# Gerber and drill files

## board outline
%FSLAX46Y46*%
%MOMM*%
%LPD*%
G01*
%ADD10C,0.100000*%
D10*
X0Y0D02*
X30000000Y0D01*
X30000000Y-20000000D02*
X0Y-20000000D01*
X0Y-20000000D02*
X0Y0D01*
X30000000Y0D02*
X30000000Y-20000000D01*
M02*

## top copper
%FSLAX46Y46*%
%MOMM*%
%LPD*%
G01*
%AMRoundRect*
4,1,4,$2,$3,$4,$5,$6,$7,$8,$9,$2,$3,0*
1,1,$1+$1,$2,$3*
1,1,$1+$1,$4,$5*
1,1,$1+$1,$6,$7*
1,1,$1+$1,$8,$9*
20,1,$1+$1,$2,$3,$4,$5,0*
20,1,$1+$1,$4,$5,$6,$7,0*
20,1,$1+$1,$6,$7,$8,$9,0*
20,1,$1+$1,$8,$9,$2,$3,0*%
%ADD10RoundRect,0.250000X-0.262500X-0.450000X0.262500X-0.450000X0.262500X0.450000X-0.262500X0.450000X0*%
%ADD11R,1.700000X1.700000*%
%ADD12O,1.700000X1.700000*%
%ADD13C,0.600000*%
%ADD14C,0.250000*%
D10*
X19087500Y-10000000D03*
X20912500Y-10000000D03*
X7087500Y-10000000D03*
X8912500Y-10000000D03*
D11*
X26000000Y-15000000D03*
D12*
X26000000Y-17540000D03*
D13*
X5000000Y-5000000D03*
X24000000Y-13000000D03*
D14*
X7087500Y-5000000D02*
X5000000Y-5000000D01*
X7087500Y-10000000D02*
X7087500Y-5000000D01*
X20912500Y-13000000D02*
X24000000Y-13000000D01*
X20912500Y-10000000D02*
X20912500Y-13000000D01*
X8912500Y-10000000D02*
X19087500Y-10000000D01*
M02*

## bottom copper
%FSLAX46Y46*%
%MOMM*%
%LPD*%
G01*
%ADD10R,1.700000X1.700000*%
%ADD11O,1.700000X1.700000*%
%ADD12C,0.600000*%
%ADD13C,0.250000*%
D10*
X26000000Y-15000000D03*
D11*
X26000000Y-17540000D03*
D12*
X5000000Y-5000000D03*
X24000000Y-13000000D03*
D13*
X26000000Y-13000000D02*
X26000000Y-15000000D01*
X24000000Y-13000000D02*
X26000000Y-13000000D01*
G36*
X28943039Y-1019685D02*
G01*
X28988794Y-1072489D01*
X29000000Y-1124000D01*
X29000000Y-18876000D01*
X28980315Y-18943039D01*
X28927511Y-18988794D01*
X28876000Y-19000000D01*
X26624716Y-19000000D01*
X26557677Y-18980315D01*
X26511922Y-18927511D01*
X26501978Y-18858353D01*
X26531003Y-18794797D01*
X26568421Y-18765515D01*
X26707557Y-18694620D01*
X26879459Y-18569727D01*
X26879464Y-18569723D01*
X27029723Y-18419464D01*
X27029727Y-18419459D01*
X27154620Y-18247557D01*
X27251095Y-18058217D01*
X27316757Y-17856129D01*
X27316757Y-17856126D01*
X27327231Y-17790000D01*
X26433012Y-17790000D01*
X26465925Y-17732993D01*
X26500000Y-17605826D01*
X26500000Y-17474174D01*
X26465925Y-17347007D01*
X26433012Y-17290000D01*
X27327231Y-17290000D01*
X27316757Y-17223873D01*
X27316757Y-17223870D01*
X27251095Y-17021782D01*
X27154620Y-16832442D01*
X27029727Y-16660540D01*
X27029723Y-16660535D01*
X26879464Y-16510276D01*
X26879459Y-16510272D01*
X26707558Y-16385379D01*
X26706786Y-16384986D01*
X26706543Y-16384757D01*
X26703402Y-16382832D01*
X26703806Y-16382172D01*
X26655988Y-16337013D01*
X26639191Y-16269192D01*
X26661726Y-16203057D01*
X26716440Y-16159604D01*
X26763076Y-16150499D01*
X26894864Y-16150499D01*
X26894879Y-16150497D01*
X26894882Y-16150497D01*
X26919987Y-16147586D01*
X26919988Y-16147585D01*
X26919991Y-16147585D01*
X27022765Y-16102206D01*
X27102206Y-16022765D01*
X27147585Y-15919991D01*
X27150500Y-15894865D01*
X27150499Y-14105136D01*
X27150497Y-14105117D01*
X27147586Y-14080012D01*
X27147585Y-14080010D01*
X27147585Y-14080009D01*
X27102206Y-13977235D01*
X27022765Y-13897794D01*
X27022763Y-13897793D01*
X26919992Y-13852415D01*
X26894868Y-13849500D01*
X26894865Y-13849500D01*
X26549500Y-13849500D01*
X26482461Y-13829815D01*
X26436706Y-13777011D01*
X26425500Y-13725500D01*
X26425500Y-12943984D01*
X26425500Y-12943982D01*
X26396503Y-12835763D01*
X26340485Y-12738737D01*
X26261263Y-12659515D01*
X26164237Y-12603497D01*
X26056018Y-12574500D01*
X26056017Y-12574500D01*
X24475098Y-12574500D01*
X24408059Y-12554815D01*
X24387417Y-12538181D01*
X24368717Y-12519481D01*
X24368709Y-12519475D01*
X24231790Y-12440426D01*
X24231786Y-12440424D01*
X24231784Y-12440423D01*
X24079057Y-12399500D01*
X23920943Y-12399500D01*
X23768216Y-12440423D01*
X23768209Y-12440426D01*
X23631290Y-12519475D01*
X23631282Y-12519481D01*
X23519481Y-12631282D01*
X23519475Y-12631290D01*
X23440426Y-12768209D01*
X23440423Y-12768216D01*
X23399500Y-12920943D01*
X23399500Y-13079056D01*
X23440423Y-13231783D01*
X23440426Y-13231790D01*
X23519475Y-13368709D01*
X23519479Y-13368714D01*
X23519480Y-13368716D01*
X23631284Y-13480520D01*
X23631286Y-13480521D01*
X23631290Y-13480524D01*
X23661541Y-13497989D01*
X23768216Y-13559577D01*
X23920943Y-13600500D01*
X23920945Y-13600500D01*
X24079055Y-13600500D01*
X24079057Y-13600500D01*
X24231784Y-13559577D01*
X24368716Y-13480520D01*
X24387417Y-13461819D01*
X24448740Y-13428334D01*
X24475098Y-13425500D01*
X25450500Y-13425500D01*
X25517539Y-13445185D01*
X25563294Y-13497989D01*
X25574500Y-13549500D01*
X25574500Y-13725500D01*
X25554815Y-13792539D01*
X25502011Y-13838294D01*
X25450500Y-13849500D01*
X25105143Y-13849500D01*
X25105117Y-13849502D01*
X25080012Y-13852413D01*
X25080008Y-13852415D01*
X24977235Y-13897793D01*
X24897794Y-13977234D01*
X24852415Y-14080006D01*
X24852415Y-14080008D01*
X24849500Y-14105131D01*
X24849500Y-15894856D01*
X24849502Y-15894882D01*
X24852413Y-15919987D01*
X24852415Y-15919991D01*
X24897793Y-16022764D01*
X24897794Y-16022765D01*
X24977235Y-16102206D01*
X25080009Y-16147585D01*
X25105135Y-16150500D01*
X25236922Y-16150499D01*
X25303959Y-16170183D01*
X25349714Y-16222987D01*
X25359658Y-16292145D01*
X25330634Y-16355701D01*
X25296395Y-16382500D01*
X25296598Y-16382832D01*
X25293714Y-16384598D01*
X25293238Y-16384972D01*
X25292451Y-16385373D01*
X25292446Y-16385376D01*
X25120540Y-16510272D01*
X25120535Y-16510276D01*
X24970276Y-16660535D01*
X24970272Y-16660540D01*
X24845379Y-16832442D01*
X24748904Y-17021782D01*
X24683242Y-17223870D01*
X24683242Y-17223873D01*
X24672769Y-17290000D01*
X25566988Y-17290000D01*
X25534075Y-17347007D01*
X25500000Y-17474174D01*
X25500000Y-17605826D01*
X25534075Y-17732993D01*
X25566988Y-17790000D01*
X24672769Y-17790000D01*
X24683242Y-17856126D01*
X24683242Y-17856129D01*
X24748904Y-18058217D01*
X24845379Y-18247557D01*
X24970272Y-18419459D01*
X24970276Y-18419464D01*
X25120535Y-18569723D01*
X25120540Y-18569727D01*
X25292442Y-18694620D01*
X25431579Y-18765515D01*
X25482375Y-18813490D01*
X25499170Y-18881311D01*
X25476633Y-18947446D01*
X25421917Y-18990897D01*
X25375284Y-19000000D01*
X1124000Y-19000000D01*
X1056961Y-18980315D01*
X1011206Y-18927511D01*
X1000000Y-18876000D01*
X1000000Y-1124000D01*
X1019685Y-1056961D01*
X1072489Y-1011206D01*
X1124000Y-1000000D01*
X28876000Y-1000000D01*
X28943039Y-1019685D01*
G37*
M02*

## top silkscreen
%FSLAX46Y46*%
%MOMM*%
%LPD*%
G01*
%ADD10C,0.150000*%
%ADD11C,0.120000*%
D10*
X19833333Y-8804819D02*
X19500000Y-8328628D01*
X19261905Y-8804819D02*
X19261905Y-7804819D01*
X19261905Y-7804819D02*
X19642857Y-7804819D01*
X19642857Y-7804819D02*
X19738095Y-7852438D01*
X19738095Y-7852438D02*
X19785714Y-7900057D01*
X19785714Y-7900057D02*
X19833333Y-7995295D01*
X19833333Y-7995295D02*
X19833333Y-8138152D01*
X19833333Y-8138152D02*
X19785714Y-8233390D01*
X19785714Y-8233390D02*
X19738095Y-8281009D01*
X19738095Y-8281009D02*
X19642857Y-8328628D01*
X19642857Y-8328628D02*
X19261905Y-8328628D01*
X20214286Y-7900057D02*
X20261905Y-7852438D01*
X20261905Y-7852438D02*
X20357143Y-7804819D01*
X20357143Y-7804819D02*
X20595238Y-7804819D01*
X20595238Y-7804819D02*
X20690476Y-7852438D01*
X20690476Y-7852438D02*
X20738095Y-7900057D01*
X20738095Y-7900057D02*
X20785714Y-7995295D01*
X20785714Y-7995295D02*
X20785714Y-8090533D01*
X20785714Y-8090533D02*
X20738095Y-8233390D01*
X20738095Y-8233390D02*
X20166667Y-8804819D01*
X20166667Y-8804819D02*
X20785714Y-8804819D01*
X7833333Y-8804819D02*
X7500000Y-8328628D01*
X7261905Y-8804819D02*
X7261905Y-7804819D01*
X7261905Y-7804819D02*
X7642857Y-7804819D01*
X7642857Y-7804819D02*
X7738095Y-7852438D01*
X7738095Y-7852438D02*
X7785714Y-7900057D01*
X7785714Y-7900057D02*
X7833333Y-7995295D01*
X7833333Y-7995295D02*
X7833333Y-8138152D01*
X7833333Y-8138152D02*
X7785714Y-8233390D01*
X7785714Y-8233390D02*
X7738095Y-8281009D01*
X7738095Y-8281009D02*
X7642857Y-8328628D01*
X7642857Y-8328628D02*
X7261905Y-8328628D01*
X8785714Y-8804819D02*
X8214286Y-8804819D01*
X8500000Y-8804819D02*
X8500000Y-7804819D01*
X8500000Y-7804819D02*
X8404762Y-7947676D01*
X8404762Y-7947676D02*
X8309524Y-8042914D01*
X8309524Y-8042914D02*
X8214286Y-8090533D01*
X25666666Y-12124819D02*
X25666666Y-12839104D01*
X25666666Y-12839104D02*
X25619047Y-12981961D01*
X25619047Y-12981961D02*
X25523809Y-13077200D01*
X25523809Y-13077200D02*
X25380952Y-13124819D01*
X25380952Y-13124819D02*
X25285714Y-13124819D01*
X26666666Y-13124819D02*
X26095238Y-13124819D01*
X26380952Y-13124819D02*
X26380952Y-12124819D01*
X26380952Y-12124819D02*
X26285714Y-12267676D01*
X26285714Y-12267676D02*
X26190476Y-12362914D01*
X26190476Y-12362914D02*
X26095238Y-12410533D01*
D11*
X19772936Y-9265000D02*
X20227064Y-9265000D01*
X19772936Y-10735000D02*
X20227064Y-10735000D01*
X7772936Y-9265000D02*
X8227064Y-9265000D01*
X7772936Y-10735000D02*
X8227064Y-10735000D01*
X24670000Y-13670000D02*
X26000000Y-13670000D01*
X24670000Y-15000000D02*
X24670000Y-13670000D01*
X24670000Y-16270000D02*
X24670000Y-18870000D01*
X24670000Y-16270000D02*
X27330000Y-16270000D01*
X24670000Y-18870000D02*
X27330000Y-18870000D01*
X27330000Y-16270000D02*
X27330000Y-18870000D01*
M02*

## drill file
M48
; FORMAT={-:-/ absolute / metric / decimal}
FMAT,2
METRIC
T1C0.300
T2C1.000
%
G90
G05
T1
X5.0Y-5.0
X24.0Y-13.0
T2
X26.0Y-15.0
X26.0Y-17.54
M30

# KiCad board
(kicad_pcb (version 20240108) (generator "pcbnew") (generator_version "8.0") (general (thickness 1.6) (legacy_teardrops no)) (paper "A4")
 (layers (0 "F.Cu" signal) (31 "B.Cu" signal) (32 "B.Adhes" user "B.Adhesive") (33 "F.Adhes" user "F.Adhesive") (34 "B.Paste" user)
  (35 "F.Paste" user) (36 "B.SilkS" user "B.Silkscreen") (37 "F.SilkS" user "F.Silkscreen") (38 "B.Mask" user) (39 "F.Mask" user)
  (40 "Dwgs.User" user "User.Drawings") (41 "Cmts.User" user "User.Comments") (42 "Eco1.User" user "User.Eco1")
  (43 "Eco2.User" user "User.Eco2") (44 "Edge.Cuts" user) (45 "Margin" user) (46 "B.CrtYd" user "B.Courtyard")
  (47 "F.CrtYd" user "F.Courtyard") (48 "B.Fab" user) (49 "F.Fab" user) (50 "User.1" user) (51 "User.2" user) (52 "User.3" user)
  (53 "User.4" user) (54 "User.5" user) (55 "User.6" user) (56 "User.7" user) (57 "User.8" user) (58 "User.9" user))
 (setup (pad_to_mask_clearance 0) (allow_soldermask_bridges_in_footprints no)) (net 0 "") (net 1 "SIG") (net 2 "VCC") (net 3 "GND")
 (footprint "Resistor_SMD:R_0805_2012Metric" (layer "F.Cu") (at 20 10)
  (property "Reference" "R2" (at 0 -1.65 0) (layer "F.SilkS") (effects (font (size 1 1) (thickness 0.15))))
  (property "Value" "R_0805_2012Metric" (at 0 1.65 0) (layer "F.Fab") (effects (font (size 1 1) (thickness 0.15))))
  (fp_line (start -0.227064 -0.735) (end 0.227064 -0.735) (stroke (width 0.12) (type solid)) (layer "F.SilkS"))
  (fp_line (start -0.227064 0.735) (end 0.227064 0.735) (stroke (width 0.12) (type solid)) (layer "F.SilkS"))
  (pad "1" smd roundrect (at -0.9125 0) (size 1.025 1.4) (layers "F.Cu" "F.Paste" "F.Mask") (roundrect_rratio 0.243902) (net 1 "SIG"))
  (pad "2" smd roundrect (at 0.9125 0) (size 1.025 1.4) (layers "F.Cu" "F.Paste" "F.Mask") (roundrect_rratio 0.243902) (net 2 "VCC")))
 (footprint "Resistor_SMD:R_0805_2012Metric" (layer "F.Cu") (at 8 10)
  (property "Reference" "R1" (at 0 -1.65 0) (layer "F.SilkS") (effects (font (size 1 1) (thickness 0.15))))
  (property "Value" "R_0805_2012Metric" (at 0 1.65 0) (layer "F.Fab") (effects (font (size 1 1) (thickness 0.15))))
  (fp_line (start -0.227064 -0.735) (end 0.227064 -0.735) (stroke (width 0.12) (type solid)) (layer "F.SilkS"))
  (fp_line (start -0.227064 0.735) (end 0.227064 0.735) (stroke (width 0.12) (type solid)) (layer "F.SilkS"))
  (pad "1" smd roundrect (at -0.9125 0) (size 1.025 1.4) (layers "F.Cu" "F.Paste" "F.Mask") (roundrect_rratio 0.243902) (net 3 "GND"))
  (pad "2" smd roundrect (at 0.9125 0) (size 1.025 1.4) (layers "F.Cu" "F.Paste" "F.Mask") (roundrect_rratio 0.243902) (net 1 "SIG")))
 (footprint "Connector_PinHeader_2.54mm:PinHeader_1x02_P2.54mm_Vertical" (layer "F.Cu") (at 26 15)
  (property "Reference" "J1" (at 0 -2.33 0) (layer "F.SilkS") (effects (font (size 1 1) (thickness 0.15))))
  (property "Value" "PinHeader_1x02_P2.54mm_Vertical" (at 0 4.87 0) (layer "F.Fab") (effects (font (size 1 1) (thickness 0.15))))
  (fp_line (start -1.33 -1.33) (end 0 -1.33) (stroke (width 0.12) (type solid)) (layer "F.SilkS"))
  (fp_line (start -1.33 0) (end -1.33 -1.33) (stroke (width 0.12) (type solid)) (layer "F.SilkS"))
  (fp_line (start -1.33 1.27) (end -1.33 3.87) (stroke (width 0.12) (type solid)) (layer "F.SilkS"))
  (fp_line (start -1.33 1.27) (end 1.33 1.27) (stroke (width 0.12) (type solid)) (layer "F.SilkS"))
  (fp_line (start -1.33 3.87) (end 1.33 3.87) (stroke (width 0.12) (type solid)) (layer "F.SilkS"))
  (fp_line (start 1.33 1.27) (end 1.33 3.87) (stroke (width 0.12) (type solid)) (layer "F.SilkS"))
  (pad "1" thru_hole rect (at 0 0) (size 1.7 1.7) (drill 1) (layers "*.Cu" "*.Mask") (remove_unused_layers no) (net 2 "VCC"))
  (pad "2" thru_hole oval (at 0 2.54) (size 1.7 1.7) (drill 1) (layers "*.Cu" "*.Mask") (remove_unused_layers no) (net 3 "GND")))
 (gr_line (start 0 0) (end 30 0) (stroke (width 0.1) (type default)) (layer "Edge.Cuts"))
 (gr_line (start 30 20) (end 0 20) (stroke (width 0.1) (type default)) (layer "Edge.Cuts"))
 (gr_line (start 0 20) (end 0 0) (stroke (width 0.1) (type default)) (layer "Edge.Cuts"))
 (gr_line (start 30 0) (end 30 20) (stroke (width 0.1) (type default)) (layer "Edge.Cuts"))
 (segment (start 7.0875 5) (end 5 5) (width 0.25) (layer "F.Cu") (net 3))
 (segment (start 7.0875 10) (end 7.0875 5) (width 0.25) (layer "F.Cu") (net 3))
 (via (at 5 5) (size 0.6) (drill 0.3) (layers "F.Cu" "B.Cu") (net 3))
 (segment (start 20.9125 13) (end 24 13) (width 0.25) (layer "F.Cu") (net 2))
 (segment (start 20.9125 10) (end 20.9125 13) (width 0.25) (layer "F.Cu") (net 2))
 (via (at 24 13) (size 0.6) (drill 0.3) (layers "F.Cu" "B.Cu") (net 2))
 (segment (start 26 13) (end 26 15) (width 0.25) (layer "B.Cu") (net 2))
 (segment (start 24 13) (end 26 13) (width 0.25) (layer "B.Cu") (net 2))
 (segment (start 8.9125 10) (end 19.0875 10) (width 0.25) (layer "F.Cu") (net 1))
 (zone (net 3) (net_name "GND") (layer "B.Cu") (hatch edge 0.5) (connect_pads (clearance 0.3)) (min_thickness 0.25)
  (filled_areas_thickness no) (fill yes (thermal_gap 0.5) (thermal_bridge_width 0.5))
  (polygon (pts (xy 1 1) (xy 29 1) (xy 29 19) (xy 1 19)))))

